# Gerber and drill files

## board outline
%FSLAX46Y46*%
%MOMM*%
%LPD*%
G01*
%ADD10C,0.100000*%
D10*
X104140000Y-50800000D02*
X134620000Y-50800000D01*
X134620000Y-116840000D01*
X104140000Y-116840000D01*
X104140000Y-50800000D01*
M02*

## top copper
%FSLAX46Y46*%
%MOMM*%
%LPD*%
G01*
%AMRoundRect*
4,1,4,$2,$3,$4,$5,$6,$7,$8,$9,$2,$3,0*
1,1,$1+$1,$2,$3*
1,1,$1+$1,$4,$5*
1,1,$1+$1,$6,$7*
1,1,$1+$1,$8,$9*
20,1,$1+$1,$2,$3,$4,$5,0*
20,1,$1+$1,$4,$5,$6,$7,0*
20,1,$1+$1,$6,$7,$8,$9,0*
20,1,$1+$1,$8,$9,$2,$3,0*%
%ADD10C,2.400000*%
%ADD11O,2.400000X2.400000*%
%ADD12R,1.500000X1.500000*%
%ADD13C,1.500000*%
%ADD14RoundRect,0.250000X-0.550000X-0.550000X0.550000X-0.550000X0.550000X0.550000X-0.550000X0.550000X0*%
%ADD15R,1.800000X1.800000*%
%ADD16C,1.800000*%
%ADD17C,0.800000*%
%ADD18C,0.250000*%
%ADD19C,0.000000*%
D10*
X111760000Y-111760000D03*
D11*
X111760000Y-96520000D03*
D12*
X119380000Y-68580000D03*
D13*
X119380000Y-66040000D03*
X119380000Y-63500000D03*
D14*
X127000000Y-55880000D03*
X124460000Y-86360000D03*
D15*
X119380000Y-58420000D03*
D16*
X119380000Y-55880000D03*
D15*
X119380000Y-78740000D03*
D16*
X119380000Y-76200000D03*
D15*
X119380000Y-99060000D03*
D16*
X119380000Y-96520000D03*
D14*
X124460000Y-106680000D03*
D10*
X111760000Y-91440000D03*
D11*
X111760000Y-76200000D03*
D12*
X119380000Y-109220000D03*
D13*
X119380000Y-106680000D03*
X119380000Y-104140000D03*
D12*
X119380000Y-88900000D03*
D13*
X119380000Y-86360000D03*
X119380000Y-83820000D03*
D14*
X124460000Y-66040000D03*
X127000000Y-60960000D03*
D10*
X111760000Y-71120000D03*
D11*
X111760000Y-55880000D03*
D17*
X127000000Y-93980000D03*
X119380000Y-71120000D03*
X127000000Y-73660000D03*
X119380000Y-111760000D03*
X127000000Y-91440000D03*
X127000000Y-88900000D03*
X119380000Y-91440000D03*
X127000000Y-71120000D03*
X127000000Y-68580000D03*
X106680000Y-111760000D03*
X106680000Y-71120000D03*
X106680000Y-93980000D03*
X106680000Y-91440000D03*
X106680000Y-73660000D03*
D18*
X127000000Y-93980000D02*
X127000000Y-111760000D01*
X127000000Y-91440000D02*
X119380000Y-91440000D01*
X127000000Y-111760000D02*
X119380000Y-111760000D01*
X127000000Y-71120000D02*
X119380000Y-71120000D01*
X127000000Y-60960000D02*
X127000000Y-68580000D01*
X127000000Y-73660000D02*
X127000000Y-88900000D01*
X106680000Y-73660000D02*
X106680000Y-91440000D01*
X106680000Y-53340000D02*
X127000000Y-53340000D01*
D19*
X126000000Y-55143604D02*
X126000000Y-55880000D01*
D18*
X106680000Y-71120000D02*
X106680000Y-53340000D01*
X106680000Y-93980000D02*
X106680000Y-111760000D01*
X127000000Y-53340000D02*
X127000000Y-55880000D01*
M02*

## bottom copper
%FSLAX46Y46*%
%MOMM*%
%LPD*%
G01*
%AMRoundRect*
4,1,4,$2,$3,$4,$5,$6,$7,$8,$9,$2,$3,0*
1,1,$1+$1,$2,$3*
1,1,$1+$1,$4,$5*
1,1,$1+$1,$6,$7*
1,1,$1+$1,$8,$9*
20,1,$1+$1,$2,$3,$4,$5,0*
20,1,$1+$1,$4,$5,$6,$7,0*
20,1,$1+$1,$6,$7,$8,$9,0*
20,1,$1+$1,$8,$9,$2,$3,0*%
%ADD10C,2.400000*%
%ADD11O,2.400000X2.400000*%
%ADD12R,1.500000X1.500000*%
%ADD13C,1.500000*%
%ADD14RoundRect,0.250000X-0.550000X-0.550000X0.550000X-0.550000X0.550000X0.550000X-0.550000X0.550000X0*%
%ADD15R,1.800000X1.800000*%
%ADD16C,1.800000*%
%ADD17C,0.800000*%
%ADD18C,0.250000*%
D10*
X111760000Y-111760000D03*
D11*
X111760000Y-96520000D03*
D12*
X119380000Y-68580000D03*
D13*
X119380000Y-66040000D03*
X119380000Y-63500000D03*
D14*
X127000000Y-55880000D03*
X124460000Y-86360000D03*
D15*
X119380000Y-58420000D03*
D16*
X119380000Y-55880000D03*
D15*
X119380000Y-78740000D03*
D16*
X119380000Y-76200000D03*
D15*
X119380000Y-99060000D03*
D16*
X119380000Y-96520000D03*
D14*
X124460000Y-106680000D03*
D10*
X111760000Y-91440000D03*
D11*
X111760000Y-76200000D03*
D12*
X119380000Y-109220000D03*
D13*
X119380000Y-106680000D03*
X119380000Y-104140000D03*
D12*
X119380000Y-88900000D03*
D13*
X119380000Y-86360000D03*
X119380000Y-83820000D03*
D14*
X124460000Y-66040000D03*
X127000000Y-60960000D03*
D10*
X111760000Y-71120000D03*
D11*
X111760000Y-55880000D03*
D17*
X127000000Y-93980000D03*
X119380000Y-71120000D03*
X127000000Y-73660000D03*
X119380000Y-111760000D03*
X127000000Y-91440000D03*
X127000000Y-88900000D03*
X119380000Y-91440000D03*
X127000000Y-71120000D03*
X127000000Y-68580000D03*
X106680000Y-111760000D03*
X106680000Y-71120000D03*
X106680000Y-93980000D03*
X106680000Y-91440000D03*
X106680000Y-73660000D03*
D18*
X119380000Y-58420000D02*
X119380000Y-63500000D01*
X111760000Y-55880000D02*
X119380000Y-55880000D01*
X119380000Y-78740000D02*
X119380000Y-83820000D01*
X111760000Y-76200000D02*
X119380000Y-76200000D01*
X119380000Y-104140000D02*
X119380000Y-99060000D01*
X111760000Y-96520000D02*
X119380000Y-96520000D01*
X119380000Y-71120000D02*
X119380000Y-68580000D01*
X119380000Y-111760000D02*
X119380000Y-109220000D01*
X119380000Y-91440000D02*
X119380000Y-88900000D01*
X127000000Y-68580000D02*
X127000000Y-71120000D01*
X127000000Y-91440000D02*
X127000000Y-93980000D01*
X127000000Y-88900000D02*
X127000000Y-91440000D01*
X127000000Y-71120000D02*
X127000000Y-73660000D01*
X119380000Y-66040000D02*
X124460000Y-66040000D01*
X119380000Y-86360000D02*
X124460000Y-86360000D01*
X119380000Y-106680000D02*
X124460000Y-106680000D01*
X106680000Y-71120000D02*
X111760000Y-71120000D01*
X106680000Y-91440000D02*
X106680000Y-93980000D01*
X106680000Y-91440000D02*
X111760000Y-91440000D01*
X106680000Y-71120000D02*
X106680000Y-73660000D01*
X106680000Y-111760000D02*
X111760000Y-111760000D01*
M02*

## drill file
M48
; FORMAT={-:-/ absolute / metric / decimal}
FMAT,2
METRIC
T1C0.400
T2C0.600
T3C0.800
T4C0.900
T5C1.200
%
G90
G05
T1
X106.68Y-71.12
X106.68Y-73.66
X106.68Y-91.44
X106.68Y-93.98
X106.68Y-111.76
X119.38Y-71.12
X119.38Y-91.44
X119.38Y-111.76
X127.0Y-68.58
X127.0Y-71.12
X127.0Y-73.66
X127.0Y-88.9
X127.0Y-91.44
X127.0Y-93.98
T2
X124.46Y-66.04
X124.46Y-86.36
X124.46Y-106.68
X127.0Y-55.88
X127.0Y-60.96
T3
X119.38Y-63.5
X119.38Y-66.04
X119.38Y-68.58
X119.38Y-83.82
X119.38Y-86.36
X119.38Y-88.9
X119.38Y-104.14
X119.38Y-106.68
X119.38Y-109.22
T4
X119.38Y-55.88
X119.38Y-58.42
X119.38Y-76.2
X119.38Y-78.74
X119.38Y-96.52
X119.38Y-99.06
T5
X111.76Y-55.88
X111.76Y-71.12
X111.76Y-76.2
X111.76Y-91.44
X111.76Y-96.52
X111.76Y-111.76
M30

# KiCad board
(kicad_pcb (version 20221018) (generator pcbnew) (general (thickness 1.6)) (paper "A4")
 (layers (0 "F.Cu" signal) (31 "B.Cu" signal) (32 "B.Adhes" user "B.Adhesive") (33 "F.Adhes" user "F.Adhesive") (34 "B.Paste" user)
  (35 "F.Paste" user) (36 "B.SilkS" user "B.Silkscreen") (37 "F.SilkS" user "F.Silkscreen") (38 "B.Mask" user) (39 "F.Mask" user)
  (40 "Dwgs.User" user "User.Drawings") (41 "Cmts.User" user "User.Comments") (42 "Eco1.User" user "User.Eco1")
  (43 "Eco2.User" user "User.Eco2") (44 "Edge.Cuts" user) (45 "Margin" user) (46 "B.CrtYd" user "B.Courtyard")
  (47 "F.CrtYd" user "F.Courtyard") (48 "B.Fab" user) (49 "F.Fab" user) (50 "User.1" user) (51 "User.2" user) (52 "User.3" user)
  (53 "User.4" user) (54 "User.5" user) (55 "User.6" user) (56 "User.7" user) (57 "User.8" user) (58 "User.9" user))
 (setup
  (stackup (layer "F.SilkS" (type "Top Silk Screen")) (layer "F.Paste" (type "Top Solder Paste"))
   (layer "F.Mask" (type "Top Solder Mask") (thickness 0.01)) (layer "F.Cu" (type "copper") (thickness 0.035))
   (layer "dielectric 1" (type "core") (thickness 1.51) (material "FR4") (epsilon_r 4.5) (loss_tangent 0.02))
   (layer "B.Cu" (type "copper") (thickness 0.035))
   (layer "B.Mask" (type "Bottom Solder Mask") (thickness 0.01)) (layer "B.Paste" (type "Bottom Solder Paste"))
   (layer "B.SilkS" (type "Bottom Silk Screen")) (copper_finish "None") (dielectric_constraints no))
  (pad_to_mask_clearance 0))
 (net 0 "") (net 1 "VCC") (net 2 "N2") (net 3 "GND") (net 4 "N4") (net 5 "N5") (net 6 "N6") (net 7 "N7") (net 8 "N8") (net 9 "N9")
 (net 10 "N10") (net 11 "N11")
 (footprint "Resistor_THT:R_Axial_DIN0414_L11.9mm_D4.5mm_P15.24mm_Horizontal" (layer "F.Cu") (at 111.76 111.76 90)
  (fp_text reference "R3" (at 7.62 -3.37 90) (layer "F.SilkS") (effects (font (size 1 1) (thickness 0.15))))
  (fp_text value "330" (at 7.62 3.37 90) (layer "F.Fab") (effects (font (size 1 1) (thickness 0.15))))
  (pad "1" thru_hole circle (at 0 0 90) (size 2.4 2.4) (drill 1.2) (layers "*.Cu" "*.Mask") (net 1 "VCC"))
  (pad "2" thru_hole oval (at 15.24 0 90) (size 2.4 2.4) (drill 1.2) (layers "*.Cu" "*.Mask") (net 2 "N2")))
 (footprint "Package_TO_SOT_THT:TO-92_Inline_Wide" (layer "F.Cu") (at 119.38 68.58 90)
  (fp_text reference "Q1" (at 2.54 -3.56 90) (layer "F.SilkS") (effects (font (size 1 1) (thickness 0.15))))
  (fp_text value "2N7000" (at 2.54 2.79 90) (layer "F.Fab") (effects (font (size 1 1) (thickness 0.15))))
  (pad "1" thru_hole rect (at 0 0 90) (size 1.5 1.5) (drill 0.8) (layers "*.Cu" "*.Mask") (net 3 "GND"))
  (pad "2" thru_hole circle (at 2.54 0 90) (size 1.5 1.5) (drill 0.8) (layers "*.Cu" "*.Mask") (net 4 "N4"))
  (pad "3" thru_hole circle (at 5.08 0 90) (size 1.5 1.5) (drill 0.8) (layers "*.Cu" "*.Mask") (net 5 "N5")))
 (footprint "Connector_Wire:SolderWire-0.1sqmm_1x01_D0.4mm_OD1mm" (layer "F.Cu") (at 127 55.88)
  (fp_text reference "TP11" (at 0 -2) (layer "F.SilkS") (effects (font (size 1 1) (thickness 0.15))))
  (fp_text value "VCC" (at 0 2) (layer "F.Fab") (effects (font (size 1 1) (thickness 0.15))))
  (pad "1" thru_hole roundrect (at 0 0) (size 1.6 1.6) (drill 0.6) (layers "*.Cu" "*.Mask") (roundrect_rratio 0.15625) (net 1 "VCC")))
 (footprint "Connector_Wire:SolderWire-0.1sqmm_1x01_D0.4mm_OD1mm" (layer "F.Cu") (at 124.46 86.36)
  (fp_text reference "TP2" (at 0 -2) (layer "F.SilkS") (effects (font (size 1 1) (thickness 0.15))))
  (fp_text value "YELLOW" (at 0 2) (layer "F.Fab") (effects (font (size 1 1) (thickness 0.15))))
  (pad "1" thru_hole roundrect (at 0 0) (size 1.6 1.6) (drill 0.6) (layers "*.Cu" "*.Mask") (roundrect_rratio 0.15625) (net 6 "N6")))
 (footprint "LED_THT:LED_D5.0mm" (layer "F.Cu") (at 119.38 58.42 90)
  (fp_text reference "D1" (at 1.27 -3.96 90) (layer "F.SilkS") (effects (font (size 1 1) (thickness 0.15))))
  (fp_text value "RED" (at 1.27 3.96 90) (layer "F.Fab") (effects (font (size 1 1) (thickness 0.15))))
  (pad "1" thru_hole rect (at 0 0 90) (size 1.8 1.8) (drill 0.9) (layers "*.Cu" "*.Mask") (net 5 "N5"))
  (pad "2" thru_hole circle (at 2.54 0 90) (size 1.8 1.8) (drill 0.9) (layers "*.Cu" "*.Mask") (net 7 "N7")))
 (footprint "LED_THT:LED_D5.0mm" (layer "F.Cu") (at 119.38 78.74 90)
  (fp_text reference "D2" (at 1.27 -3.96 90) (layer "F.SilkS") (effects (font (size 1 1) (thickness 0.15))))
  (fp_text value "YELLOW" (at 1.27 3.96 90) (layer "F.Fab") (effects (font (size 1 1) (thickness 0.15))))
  (pad "1" thru_hole rect (at 0 0 90) (size 1.8 1.8) (drill 0.9) (layers "*.Cu" "*.Mask") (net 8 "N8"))
  (pad "2" thru_hole circle (at 2.54 0 90) (size 1.8 1.8) (drill 0.9) (layers "*.Cu" "*.Mask") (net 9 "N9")))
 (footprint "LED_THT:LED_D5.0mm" (layer "F.Cu") (at 119.38 99.06 90)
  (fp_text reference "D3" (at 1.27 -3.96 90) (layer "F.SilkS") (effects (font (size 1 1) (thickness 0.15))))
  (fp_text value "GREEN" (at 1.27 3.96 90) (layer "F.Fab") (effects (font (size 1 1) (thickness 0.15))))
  (pad "1" thru_hole rect (at 0 0 90) (size 1.8 1.8) (drill 0.9) (layers "*.Cu" "*.Mask") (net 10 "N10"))
  (pad "2" thru_hole circle (at 2.54 0 90) (size 1.8 1.8) (drill 0.9) (layers "*.Cu" "*.Mask") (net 2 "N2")))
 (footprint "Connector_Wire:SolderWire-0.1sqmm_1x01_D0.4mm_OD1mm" (layer "F.Cu") (at 124.46 106.68)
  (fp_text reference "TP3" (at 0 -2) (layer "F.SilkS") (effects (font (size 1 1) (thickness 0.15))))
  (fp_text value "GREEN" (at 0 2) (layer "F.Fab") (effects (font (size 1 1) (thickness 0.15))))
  (pad "1" thru_hole roundrect (at 0 0) (size 1.6 1.6) (drill 0.6) (layers "*.Cu" "*.Mask") (roundrect_rratio 0.15625) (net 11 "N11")))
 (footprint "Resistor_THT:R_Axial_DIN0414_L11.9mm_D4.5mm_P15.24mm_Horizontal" (layer "F.Cu") (at 111.76 91.44 90)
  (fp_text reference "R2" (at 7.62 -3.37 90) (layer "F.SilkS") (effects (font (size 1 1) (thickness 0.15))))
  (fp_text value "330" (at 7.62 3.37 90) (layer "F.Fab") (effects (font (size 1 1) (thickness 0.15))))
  (pad "1" thru_hole circle (at 0 0 90) (size 2.4 2.4) (drill 1.2) (layers "*.Cu" "*.Mask") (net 1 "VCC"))
  (pad "2" thru_hole oval (at 15.24 0 90) (size 2.4 2.4) (drill 1.2) (layers "*.Cu" "*.Mask") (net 9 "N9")))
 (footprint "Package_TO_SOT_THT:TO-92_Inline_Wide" (layer "F.Cu") (at 119.38 109.22 90)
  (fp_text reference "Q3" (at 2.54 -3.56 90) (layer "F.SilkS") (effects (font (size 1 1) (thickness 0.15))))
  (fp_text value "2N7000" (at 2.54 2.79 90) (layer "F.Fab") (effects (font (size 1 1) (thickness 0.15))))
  (pad "1" thru_hole rect (at 0 0 90) (size 1.5 1.5) (drill 0.8) (layers "*.Cu" "*.Mask") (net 3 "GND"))
  (pad "2" thru_hole circle (at 2.54 0 90) (size 1.5 1.5) (drill 0.8) (layers "*.Cu" "*.Mask") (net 11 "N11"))
  (pad "3" thru_hole circle (at 5.08 0 90) (size 1.5 1.5) (drill 0.8) (layers "*.Cu" "*.Mask") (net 10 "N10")))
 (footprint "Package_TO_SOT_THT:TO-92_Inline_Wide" (layer "F.Cu") (at 119.38 88.9 90)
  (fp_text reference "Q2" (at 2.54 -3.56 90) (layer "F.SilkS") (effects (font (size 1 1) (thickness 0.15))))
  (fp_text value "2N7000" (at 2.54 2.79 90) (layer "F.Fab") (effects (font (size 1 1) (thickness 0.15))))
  (pad "1" thru_hole rect (at 0 0 90) (size 1.5 1.5) (drill 0.8) (layers "*.Cu" "*.Mask") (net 3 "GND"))
  (pad "2" thru_hole circle (at 2.54 0 90) (size 1.5 1.5) (drill 0.8) (layers "*.Cu" "*.Mask") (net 6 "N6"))
  (pad "3" thru_hole circle (at 5.08 0 90) (size 1.5 1.5) (drill 0.8) (layers "*.Cu" "*.Mask") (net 8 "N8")))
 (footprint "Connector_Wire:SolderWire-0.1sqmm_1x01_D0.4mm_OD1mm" (layer "F.Cu") (at 124.46 66.04)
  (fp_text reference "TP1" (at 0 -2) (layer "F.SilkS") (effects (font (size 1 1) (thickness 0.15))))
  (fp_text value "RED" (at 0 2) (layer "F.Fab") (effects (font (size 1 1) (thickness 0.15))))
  (pad "1" thru_hole roundrect (at 0 0) (size 1.6 1.6) (drill 0.6) (layers "*.Cu" "*.Mask") (roundrect_rratio 0.15625) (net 4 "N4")))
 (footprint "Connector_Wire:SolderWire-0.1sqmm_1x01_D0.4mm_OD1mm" (layer "F.Cu") (at 127 60.96)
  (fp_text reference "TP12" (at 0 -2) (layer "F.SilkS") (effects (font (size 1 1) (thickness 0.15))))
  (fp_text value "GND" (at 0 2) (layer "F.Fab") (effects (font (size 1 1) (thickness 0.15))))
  (pad "1" thru_hole roundrect (at 0 0) (size 1.6 1.6) (drill 0.6) (layers "*.Cu" "*.Mask") (roundrect_rratio 0.15625) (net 3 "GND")))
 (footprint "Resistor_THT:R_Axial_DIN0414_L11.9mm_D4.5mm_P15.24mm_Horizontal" (layer "F.Cu") (at 111.76 71.12 90)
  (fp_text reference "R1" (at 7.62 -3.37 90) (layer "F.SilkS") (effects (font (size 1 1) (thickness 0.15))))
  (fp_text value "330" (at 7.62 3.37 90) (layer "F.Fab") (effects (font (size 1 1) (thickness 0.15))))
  (pad "1" thru_hole circle (at 0 0 90) (size 2.4 2.4) (drill 1.2) (layers "*.Cu" "*.Mask") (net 1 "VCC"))
  (pad "2" thru_hole oval (at 15.24 0 90) (size 2.4 2.4) (drill 1.2) (layers "*.Cu" "*.Mask") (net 7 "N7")))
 (gr_rect (start 104.14 50.8) (end 134.62 116.84) (stroke (width 0.1) (type default)) (fill none) (layer "Edge.Cuts"))
 (segment (start 119.38 58.42) (end 119.38 63.5) (width 0.25) (layer "B.Cu") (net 5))
 (segment (start 111.76 55.88) (end 119.38 55.88) (width 0.25) (layer "B.Cu") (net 7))
 (segment (start 119.38 78.74) (end 119.38 83.82) (width 0.25) (layer "B.Cu") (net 8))
 (segment (start 111.76 76.2) (end 119.38 76.2) (width 0.25) (layer "B.Cu") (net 9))
 (segment (start 119.38 104.14) (end 119.38 99.06) (width 0.25) (layer "B.Cu") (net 10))
 (segment (start 111.76 96.52) (end 119.38 96.52) (width 0.25) (layer "B.Cu") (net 2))
 (segment (start 127 93.98) (end 127 111.76) (width 0.25) (layer "F.Cu") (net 3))
 (segment (start 127 91.44) (end 119.38 91.44) (width 0.25) (layer "F.Cu") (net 3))
 (segment (start 127 111.76) (end 119.38 111.76) (width 0.25) (layer "F.Cu") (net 3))
 (segment (start 127 71.12) (end 119.38 71.12) (width 0.25) (layer "F.Cu") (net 3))
 (segment (start 127 60.96) (end 127 68.58) (width 0.25) (layer "F.Cu") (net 3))
 (segment (start 127 73.66) (end 127 88.9) (width 0.25) (layer "F.Cu") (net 3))
 (via (at 127 93.98) (size 0.8) (drill 0.4) (layers "F.Cu" "B.Cu") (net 3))
 (via (at 119.38 71.12) (size 0.8) (drill 0.4) (layers "F.Cu" "B.Cu") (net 3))
 (via (at 127 73.66) (size 0.8) (drill 0.4) (layers "F.Cu" "B.Cu") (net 3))
 (via (at 119.38 111.76) (size 0.8) (drill 0.4) (layers "F.Cu" "B.Cu") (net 3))
 (via (at 127 91.44) (size 0.8) (drill 0.4) (layers "F.Cu" "B.Cu") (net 3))
 (via (at 127 88.9) (size 0.8) (drill 0.4) (layers "F.Cu" "B.Cu") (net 3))
 (via (at 119.38 91.44) (size 0.8) (drill 0.4) (layers "F.Cu" "B.Cu") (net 3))
 (via (at 127 71.12) (size 0.8) (drill 0.4) (layers "F.Cu" "B.Cu") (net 3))
 (via (at 127 68.58) (size 0.8) (drill 0.4) (layers "F.Cu" "B.Cu") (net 3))
 (segment (start 119.38 71.12) (end 119.38 68.58) (width 0.25) (layer "B.Cu") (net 3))
 (segment (start 119.38 111.76) (end 119.38 109.22) (width 0.25) (layer "B.Cu") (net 3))
 (segment (start 119.38 91.44) (end 119.38 88.9) (width 0.25) (layer "B.Cu") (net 3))
 (segment (start 127 68.58) (end 127 71.12) (width 0.25) (layer "B.Cu") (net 3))
 (segment (start 127 91.44) (end 127 93.98) (width 0.25) (layer "B.Cu") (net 3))
 (segment (start 127 88.9) (end 127 91.44) (width 0.25) (layer "B.Cu") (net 3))
 (segment (start 127 71.12) (end 127 73.66) (width 0.25) (layer "B.Cu") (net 3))
 (segment (start 119.38 66.04) (end 124.46 66.04) (width 0.25) (layer "B.Cu") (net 4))
 (segment (start 119.38 86.36) (end 124.46 86.36) (width 0.25) (layer "B.Cu") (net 6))
 (segment (start 119.38 106.68) (end 124.46 106.68) (width 0.25) (layer "B.Cu") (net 11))
 (segment (start 106.68 73.66) (end 106.68 91.44) (width 0.25) (layer "F.Cu") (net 1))
 (segment (start 106.68 53.34) (end 127 53.34) (width 0.25) (layer "F.Cu") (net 1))
 (segment (start 126 55.143604) (end 126 55.88) (width 0) (layer "F.Cu") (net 1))
 (segment (start 106.68 71.12) (end 106.68 53.34) (width 0.25) (layer "F.Cu") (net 1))
 (segment (start 106.68 93.98) (end 106.68 111.76) (width 0.25) (layer "F.Cu") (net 1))
 (segment (start 127 53.34) (end 127 55.88) (width 0.25) (layer "F.Cu") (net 1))
 (via (at 106.68 111.76) (size 0.8) (drill 0.4) (layers "F.Cu" "B.Cu") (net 1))
 (via (at 106.68 71.12) (size 0.8) (drill 0.4) (layers "F.Cu" "B.Cu") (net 1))
 (via (at 106.68 93.98) (size 0.8) (drill 0.4) (layers "F.Cu" "B.Cu") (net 1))
 (via (at 106.68 91.44) (size 0.8) (drill 0.4) (layers "F.Cu" "B.Cu") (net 1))
 (via (at 106.68 73.66) (size 0.8) (drill 0.4) (layers "F.Cu" "B.Cu") (free) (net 1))
 (segment (start 106.68 71.12) (end 111.76 71.12) (width 0.25) (layer "B.Cu") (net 1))
 (segment (start 106.68 91.44) (end 106.68 93.98) (width 0.25) (layer "B.Cu") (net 1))
 (segment (start 106.68 91.44) (end 111.76 91.44) (width 0.25) (layer "B.Cu") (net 1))
 (segment (start 106.68 71.12) (end 106.68 73.66) (width 0.25) (layer "B.Cu") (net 1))
 (segment (start 106.68 111.76) (end 111.76 111.76) (width 0.25) (layer "B.Cu") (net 1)))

